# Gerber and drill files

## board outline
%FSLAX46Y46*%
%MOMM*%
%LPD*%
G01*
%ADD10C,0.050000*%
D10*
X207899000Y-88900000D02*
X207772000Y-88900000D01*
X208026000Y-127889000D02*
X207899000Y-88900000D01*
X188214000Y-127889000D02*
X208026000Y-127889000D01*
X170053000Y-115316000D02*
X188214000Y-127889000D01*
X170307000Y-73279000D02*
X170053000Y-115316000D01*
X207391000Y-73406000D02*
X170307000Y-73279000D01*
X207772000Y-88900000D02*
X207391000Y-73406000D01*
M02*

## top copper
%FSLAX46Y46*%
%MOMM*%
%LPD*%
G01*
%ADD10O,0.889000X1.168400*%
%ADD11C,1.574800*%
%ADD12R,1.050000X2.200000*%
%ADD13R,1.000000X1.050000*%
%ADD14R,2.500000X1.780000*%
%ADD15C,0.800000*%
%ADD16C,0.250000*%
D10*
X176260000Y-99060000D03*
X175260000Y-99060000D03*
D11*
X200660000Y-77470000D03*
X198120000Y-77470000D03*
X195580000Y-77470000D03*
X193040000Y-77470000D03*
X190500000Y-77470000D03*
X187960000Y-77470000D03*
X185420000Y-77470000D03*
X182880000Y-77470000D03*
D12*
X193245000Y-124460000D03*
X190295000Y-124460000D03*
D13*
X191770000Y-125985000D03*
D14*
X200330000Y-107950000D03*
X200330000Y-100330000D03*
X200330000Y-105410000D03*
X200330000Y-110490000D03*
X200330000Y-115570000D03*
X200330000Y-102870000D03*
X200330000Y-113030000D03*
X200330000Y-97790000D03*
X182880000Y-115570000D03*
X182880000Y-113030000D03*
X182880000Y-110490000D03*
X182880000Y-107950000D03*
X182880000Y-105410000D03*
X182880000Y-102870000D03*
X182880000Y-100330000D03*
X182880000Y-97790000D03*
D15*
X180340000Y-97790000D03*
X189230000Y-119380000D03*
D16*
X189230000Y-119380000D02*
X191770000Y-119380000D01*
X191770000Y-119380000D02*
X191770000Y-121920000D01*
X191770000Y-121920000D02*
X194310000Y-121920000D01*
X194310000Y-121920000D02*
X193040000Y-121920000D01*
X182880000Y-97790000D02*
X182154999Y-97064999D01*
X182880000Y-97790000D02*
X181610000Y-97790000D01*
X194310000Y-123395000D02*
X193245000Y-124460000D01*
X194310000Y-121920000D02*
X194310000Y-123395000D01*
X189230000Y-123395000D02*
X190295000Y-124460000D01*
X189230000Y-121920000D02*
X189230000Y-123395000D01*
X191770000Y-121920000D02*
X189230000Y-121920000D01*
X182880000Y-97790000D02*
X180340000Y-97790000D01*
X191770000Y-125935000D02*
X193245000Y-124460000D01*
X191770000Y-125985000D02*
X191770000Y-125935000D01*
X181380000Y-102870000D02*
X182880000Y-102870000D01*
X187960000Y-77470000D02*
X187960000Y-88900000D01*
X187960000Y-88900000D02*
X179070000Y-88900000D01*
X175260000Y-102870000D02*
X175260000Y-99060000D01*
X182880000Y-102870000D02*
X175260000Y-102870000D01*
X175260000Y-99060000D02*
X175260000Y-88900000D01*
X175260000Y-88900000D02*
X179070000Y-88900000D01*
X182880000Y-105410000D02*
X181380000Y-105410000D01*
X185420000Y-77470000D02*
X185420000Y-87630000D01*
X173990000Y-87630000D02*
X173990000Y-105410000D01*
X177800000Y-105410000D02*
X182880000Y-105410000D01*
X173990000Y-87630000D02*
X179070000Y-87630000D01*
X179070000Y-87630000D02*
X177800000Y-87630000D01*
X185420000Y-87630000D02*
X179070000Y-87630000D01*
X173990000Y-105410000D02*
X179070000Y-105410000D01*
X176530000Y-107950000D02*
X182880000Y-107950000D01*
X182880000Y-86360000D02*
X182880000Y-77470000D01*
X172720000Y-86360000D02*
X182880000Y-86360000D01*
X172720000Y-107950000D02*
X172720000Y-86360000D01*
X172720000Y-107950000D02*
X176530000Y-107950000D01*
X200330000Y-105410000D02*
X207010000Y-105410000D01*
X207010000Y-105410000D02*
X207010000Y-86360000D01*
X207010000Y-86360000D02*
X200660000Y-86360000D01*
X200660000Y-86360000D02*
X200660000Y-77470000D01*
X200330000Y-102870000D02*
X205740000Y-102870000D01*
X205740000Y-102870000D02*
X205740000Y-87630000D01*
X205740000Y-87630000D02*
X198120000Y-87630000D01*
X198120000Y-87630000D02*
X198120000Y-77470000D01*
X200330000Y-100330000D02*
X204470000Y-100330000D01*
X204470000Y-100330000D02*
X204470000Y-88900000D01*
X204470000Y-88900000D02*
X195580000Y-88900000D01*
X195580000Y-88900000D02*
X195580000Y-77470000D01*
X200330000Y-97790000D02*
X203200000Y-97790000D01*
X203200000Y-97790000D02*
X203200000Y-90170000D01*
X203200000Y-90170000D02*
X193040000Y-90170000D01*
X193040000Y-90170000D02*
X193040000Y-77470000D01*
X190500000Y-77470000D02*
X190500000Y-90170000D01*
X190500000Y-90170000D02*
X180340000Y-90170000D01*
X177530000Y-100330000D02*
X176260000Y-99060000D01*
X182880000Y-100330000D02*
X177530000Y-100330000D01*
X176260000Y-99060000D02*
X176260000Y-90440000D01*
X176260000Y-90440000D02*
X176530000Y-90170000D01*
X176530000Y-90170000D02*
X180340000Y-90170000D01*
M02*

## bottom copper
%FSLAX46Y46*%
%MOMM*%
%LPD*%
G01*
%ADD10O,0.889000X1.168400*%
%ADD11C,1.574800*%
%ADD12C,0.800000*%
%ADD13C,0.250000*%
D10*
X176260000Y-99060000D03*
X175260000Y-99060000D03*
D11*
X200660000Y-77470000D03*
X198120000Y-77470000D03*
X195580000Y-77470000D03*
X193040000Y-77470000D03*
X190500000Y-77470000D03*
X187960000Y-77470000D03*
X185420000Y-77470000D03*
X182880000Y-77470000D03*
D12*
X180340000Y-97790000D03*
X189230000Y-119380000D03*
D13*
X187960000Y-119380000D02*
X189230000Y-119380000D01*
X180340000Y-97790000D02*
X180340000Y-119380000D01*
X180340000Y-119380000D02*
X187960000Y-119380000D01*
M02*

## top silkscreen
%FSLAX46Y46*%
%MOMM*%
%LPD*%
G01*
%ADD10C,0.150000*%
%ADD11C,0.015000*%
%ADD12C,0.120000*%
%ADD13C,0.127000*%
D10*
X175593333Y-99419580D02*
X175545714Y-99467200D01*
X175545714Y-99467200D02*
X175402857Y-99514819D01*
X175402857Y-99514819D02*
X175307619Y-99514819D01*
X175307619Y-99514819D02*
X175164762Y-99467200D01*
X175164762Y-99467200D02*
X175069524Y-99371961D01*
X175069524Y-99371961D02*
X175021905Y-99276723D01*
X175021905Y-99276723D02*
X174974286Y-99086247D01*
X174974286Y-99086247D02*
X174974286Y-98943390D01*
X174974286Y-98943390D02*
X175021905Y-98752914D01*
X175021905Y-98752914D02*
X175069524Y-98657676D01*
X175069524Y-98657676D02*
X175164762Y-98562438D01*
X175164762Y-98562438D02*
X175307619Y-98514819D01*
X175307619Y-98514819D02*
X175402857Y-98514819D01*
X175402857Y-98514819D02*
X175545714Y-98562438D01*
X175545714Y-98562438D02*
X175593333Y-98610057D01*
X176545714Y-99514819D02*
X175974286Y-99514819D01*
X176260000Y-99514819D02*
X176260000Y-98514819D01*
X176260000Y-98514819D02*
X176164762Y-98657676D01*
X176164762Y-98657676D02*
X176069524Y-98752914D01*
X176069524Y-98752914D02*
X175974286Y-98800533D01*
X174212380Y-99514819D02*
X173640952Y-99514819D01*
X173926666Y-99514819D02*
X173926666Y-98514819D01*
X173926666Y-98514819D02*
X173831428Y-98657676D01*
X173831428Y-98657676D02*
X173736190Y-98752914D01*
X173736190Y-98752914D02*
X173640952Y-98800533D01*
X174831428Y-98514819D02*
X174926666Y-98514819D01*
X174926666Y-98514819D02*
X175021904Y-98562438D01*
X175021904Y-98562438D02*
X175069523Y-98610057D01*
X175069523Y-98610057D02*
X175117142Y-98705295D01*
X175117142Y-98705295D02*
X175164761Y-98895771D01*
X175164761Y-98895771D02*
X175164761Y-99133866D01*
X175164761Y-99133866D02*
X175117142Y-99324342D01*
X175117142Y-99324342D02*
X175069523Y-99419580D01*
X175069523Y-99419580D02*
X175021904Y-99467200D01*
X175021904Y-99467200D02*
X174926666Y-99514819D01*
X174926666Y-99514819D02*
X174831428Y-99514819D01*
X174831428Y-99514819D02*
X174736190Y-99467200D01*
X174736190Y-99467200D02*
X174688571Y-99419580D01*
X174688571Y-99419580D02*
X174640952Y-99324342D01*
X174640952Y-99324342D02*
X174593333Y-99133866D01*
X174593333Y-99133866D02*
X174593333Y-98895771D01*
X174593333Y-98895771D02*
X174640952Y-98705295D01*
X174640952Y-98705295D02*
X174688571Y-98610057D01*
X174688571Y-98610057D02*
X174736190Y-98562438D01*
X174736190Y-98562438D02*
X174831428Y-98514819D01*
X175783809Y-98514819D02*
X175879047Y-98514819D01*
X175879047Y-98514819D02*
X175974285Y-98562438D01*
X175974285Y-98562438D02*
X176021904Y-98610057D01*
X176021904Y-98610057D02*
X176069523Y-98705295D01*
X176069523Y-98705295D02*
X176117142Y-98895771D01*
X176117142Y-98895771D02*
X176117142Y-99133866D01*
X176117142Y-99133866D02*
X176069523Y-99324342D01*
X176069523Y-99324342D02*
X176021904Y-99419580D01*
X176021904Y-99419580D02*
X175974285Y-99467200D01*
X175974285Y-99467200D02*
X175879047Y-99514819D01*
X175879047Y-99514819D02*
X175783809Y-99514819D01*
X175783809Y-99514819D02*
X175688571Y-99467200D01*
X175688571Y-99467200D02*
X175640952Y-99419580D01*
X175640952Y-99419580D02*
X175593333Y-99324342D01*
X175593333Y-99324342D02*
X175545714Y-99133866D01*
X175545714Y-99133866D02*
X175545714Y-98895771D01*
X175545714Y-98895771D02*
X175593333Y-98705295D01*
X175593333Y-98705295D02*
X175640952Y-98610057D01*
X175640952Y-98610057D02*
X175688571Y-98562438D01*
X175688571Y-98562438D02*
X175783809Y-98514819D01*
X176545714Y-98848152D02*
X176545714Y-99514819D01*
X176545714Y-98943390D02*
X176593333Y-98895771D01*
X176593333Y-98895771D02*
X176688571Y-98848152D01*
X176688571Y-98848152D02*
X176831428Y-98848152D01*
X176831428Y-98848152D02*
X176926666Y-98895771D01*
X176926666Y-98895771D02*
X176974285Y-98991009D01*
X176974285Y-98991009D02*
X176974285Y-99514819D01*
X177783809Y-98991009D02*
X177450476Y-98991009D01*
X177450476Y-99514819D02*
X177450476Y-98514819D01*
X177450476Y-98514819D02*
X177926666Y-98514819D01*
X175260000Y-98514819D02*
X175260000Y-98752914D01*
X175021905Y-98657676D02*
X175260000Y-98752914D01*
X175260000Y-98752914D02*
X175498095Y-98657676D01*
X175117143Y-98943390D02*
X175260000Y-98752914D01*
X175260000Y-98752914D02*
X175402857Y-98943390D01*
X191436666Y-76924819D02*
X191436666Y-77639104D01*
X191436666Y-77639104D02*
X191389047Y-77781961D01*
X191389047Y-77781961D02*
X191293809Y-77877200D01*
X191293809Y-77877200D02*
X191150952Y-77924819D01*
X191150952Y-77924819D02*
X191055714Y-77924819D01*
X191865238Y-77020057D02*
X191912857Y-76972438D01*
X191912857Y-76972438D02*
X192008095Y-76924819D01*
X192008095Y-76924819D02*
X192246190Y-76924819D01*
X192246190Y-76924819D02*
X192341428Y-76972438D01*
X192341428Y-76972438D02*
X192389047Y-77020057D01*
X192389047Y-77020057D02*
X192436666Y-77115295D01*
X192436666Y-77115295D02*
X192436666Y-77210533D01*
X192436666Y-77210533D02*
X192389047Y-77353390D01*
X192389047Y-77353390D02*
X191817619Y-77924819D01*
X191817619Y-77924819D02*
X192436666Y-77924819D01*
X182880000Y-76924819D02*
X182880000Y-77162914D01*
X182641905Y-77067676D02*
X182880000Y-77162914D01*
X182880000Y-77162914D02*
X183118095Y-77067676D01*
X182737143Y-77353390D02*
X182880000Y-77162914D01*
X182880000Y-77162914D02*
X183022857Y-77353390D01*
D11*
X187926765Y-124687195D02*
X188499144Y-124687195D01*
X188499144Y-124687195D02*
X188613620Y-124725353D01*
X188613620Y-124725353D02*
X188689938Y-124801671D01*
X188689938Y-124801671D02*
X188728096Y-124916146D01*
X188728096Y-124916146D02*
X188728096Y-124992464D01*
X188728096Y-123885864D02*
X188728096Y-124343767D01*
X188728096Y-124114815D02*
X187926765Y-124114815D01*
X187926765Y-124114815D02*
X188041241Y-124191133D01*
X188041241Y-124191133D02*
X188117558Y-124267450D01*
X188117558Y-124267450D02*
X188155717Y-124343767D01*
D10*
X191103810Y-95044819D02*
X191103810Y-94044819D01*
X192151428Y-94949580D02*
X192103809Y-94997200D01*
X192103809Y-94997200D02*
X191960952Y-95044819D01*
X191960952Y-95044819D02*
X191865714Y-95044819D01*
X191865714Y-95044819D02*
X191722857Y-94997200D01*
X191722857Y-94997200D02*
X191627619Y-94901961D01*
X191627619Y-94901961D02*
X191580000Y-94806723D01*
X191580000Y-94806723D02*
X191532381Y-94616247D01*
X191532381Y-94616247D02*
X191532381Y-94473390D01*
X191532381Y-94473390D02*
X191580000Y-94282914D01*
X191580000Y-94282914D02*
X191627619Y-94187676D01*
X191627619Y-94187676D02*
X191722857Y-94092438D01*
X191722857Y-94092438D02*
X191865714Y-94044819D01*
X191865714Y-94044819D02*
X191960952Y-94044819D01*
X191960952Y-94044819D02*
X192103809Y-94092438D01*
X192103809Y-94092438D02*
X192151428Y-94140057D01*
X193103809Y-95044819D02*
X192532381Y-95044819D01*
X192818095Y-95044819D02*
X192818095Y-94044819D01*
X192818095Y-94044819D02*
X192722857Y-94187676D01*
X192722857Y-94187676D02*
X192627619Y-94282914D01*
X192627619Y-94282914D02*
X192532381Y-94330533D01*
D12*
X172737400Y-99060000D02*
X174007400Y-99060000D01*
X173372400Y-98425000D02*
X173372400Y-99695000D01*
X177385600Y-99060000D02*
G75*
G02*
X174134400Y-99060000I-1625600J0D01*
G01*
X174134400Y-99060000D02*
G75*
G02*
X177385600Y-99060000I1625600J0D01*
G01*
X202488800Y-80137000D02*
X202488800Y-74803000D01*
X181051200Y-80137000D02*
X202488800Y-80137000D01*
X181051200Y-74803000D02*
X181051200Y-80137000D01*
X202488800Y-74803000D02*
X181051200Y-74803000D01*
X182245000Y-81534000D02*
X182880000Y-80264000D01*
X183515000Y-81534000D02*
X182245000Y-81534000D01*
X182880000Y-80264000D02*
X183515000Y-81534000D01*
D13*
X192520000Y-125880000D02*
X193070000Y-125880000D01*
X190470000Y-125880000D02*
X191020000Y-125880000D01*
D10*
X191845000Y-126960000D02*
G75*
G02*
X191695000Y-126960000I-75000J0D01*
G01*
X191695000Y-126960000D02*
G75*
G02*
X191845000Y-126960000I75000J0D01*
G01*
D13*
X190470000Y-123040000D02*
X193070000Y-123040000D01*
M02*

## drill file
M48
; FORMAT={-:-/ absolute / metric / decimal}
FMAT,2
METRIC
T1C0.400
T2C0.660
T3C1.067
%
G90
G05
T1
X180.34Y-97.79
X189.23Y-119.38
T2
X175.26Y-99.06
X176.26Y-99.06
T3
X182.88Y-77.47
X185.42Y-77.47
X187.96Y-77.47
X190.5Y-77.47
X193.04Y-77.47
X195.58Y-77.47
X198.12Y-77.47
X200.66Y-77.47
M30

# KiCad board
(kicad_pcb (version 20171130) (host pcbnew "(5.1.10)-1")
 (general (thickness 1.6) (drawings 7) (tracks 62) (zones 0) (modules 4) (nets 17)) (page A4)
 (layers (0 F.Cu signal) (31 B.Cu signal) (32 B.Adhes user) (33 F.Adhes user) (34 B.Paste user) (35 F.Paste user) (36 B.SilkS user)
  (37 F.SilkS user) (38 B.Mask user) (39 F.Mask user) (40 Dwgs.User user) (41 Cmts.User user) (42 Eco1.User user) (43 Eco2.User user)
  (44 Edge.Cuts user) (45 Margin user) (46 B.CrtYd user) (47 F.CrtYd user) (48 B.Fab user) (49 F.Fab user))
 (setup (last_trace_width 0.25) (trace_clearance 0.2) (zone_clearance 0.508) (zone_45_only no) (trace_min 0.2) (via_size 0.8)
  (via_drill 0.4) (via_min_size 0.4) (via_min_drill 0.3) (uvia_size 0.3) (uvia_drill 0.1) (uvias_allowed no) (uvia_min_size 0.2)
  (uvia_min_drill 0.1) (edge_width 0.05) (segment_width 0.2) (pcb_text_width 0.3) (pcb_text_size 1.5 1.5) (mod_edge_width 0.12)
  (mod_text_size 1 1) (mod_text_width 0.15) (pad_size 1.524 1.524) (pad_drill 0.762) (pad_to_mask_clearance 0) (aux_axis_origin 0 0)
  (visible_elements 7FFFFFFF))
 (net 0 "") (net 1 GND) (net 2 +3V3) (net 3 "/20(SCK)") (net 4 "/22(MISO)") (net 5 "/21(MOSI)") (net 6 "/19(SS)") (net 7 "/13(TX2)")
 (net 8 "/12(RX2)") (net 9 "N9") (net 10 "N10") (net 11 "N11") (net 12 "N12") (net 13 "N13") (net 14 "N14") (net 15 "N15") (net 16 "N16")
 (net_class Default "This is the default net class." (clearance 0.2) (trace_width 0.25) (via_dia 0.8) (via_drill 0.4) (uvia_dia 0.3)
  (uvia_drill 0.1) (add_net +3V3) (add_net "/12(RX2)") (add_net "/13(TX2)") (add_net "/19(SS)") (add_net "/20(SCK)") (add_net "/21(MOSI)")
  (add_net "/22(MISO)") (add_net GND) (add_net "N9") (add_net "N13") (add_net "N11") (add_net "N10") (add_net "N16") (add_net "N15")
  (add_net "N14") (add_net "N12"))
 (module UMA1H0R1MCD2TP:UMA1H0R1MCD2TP (layer F.Cu) (at 175.26 99.06)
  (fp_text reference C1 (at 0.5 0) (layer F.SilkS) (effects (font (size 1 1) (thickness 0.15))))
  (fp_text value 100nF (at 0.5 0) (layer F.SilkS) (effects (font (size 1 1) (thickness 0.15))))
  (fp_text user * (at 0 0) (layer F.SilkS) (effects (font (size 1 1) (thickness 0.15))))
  (fp_line (start -2.5226 0) (end -1.2526 0) (layer F.SilkS) (width 0.12))
  (fp_line (start -1.8876 -0.635) (end -1.8876 0.635) (layer F.SilkS) (width 0.12))
  (fp_circle (center 0.5 0) (end 2.1256 0) (layer F.SilkS) (width 0.12))
  (pad 2 thru_hole oval (at 1 0) (size 0.889 1.1684) (drill 0.6604) (layers *.Cu *.Mask) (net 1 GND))
  (pad 1 thru_hole oval (at 0 0) (size 0.889 1.1684) (drill 0.6604) (layers *.Cu *.Mask) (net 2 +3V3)))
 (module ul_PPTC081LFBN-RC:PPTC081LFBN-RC (layer F.Cu) (at 182.88 77.47 180)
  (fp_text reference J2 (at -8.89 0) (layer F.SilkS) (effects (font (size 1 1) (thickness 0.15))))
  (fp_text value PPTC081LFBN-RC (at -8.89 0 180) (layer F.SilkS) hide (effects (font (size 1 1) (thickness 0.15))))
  (fp_line (start -19.6088 -2.667) (end -19.6088 2.667) (layer F.SilkS) (width 0.12))
  (fp_line (start 1.8288 -2.667) (end -19.6088 -2.667) (layer F.SilkS) (width 0.12))
  (fp_line (start 1.8288 2.667) (end 1.8288 -2.667) (layer F.SilkS) (width 0.12))
  (fp_line (start -19.6088 2.667) (end 1.8288 2.667) (layer F.SilkS) (width 0.12))
  (fp_line (start 0.635 -4.064) (end 0 -2.794) (layer F.SilkS) (width 0.12))
  (fp_line (start -0.635 -4.064) (end 0.635 -4.064) (layer F.SilkS) (width 0.12))
  (fp_line (start 0 -2.794) (end -0.635 -4.064) (layer F.SilkS) (width 0.12))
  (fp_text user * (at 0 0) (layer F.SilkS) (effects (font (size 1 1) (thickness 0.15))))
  (pad 8 thru_hole circle (at -17.78 0 180) (size 1.5748 1.5748) (drill 1.0668) (layers *.Cu *.Mask) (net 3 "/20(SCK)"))
  (pad 7 thru_hole circle (at -15.24 0 180) (size 1.5748 1.5748) (drill 1.0668) (layers *.Cu *.Mask) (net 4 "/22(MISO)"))
  (pad 6 thru_hole circle (at -12.7 0 180) (size 1.5748 1.5748) (drill 1.0668) (layers *.Cu *.Mask) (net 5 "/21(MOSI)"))
  (pad 5 thru_hole circle (at -10.16 0 180) (size 1.5748 1.5748) (drill 1.0668) (layers *.Cu *.Mask) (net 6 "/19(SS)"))
  (pad 4 thru_hole circle (at -7.62 0 180) (size 1.5748 1.5748) (drill 1.0668) (layers *.Cu *.Mask) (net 1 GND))
  (pad 3 thru_hole circle (at -5.08 0 180) (size 1.5748 1.5748) (drill 1.0668) (layers *.Cu *.Mask) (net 2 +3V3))
  (pad 2 thru_hole circle (at -2.54 0 180) (size 1.5748 1.5748) (drill 1.0668) (layers *.Cu *.Mask) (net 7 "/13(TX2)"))
  (pad 1 thru_hole circle (at 0 0 180) (size 1.5748 1.5748) (drill 1.0668) (layers *.Cu *.Mask) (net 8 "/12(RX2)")))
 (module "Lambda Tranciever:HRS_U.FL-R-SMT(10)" (layer F.Cu) (at 191.77 124.46 90)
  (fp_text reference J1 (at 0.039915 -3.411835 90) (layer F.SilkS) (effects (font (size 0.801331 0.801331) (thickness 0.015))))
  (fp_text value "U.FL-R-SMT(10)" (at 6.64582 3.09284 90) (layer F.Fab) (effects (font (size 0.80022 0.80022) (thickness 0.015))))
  (fp_line (start -1.42 0.75) (end -1.42 1.3) (layer F.SilkS) (width 0.127))
  (fp_line (start -1.42 -1.3) (end -1.42 -0.75) (layer F.SilkS) (width 0.127))
  (fp_circle (center -2.5 0) (end -2.425 0) (layer F.SilkS) (width 0.15))
  (fp_line (start 1.42 -1.3) (end 1.42 1.3) (layer F.SilkS) (width 0.127))
  (pad 3 smd rect (at 0 1.475 90) (size 2.2 1.05) (layers F.Cu F.Paste F.Mask) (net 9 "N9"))
  (pad 2 smd rect (at 0 -1.475 90) (size 2.2 1.05) (layers F.Cu F.Paste F.Mask) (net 9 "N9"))
  (pad 1 smd rect (at -1.525 0 90) (size 1.05 1) (layers F.Cu F.Paste F.Mask) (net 9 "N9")))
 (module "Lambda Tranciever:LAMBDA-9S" (layer F.Cu) (at 182.88 97.79)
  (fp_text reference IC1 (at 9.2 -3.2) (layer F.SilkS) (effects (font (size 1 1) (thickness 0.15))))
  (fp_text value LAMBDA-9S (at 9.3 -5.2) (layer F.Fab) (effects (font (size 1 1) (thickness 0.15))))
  (pad 12 smd rect (at 17.45 10.16) (size 2.5 1.78) (layers F.Cu F.Paste F.Mask) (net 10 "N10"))
  (pad 15 smd rect (at 17.45 2.54) (size 2.5 1.78) (layers F.Cu F.Paste F.Mask) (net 5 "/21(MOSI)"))
  (pad 13 smd rect (at 17.45 7.62) (size 2.5 1.78) (layers F.Cu F.Paste F.Mask) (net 3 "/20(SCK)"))
  (pad 11 smd rect (at 17.45 12.7) (size 2.5 1.78) (layers F.Cu F.Paste F.Mask) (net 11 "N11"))
  (pad 9 smd rect (at 17.45 17.78) (size 2.5 1.78) (layers F.Cu F.Paste F.Mask) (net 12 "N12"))
  (pad 14 smd rect (at 17.45 5.08) (size 2.5 1.78) (layers F.Cu F.Paste F.Mask) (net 4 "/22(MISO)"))
  (pad 10 smd rect (at 17.45 15.24) (size 2.5 1.78) (layers F.Cu F.Paste F.Mask) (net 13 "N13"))
  (pad 16 smd rect (at 17.45 0) (size 2.5 1.78) (layers F.Cu F.Paste F.Mask) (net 6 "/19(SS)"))
  (pad 8 smd rect (at 0 17.78) (size 2.5 1.78) (layers F.Cu F.Paste F.Mask) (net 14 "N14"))
  (pad 7 smd rect (at 0 15.24) (size 2.5 1.78) (layers F.Cu F.Paste F.Mask) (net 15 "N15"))
  (pad 6 smd rect (at 0 12.7) (size 2.5 1.78) (layers F.Cu F.Paste F.Mask) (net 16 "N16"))
  (pad 5 smd rect (at 0 10.16) (size 2.5 1.78) (layers F.Cu F.Paste F.Mask) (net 8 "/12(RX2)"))
  (pad 4 smd rect (at 0 7.62) (size 2.5 1.78) (layers F.Cu F.Paste F.Mask) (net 7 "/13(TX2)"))
  (pad 3 smd rect (at 0 5.08) (size 2.5 1.78) (layers F.Cu F.Paste F.Mask) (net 2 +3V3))
  (pad 2 smd rect (at 0 2.54) (size 2.5 1.78) (layers F.Cu F.Paste F.Mask) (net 1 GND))
  (pad 1 smd rect (at 0 0) (size 2.5 1.78) (layers F.Cu F.Paste F.Mask) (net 9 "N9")))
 (gr_line (start 207.899 88.9) (end 207.772 88.9) (layer Edge.Cuts) (width 0.05))
 (gr_line (start 208.026 127.889) (end 207.899 88.9) (layer Edge.Cuts) (width 0.05))
 (gr_line (start 188.214 127.889) (end 208.026 127.889) (layer Edge.Cuts) (width 0.05))
 (gr_line (start 170.053 115.316) (end 188.214 127.889) (layer Edge.Cuts) (width 0.05))
 (gr_line (start 170.307 73.279) (end 170.053 115.316) (layer Edge.Cuts) (width 0.05))
 (gr_line (start 207.391 73.406) (end 170.307 73.279) (layer Edge.Cuts) (width 0.05))
 (gr_line (start 207.772 88.9) (end 207.391 73.406) (layer Edge.Cuts) (width 0.05))
 (via (at 180.34 97.79) (size 0.8) (drill 0.4) (layers F.Cu B.Cu) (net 9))
 (via (at 189.23 119.38) (size 0.8) (drill 0.4) (layers F.Cu B.Cu) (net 9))
 (segment (start 189.23 119.38) (end 191.77 119.38) (width 0.25) (layer F.Cu) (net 9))
 (segment (start 191.77 119.38) (end 191.77 121.92) (width 0.25) (layer F.Cu) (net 9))
 (segment (start 191.77 121.92) (end 194.31 121.92) (width 0.25) (layer F.Cu) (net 9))
 (segment (start 194.31 121.92) (end 193.04 121.92) (width 0.25) (layer F.Cu) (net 9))
 (segment (start 182.88 97.79) (end 182.154999 97.064999) (width 0.25) (layer F.Cu) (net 9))
 (segment (start 182.88 97.79) (end 181.61 97.79) (width 0.25) (layer F.Cu) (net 9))
 (segment (start 187.96 119.38) (end 189.23 119.38) (width 0.25) (layer B.Cu) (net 9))
 (segment (start 194.31 123.395) (end 193.245 124.46) (width 0.25) (layer F.Cu) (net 9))
 (segment (start 194.31 121.92) (end 194.31 123.395) (width 0.25) (layer F.Cu) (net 9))
 (segment (start 189.23 123.395) (end 190.295 124.46) (width 0.25) (layer F.Cu) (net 9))
 (segment (start 189.23 121.92) (end 189.23 123.395) (width 0.25) (layer F.Cu) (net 9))
 (segment (start 191.77 121.92) (end 189.23 121.92) (width 0.25) (layer F.Cu) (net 9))
 (segment (start 182.88 97.79) (end 180.34 97.79) (width 0.25) (layer F.Cu) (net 9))
 (segment (start 180.34 97.79) (end 180.34 119.38) (width 0.25) (layer B.Cu) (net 9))
 (segment (start 180.34 119.38) (end 187.96 119.38) (width 0.25) (layer B.Cu) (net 9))
 (segment (start 191.77 125.935) (end 193.245 124.46) (width 0.25) (layer F.Cu) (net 9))
 (segment (start 191.77 125.985) (end 191.77 125.935) (width 0.25) (layer F.Cu) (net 9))
 (segment (start 181.38 102.87) (end 182.88 102.87) (width 0.25) (layer F.Cu) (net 2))
 (segment (start 187.96 77.47) (end 187.96 88.9) (width 0.25) (layer F.Cu) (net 2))
 (segment (start 187.96 88.9) (end 179.07 88.9) (width 0.25) (layer F.Cu) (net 2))
 (segment (start 175.26 102.87) (end 175.26 99.06) (width 0.25) (layer F.Cu) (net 2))
 (segment (start 182.88 102.87) (end 175.26 102.87) (width 0.25) (layer F.Cu) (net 2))
 (segment (start 175.26 99.06) (end 175.26 88.9) (width 0.25) (layer F.Cu) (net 2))
 (segment (start 175.26 88.9) (end 179.07 88.9) (width 0.25) (layer F.Cu) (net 2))
 (segment (start 182.88 105.41) (end 181.38 105.41) (width 0.25) (layer F.Cu) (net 7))
 (segment (start 185.42 77.47) (end 185.42 87.63) (width 0.25) (layer F.Cu) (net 7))
 (segment (start 173.99 87.63) (end 173.99 105.41) (width 0.25) (layer F.Cu) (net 7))
 (segment (start 177.8 105.41) (end 182.88 105.41) (width 0.25) (layer F.Cu) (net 7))
 (segment (start 173.99 87.63) (end 179.07 87.63) (width 0.25) (layer F.Cu) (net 7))
 (segment (start 179.07 87.63) (end 177.8 87.63) (width 0.25) (layer F.Cu) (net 7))
 (segment (start 185.42 87.63) (end 179.07 87.63) (width 0.25) (layer F.Cu) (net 7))
 (segment (start 173.99 105.41) (end 179.07 105.41) (width 0.25) (layer F.Cu) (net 7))
 (segment (start 176.53 107.95) (end 182.88 107.95) (width 0.25) (layer F.Cu) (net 8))
 (segment (start 182.88 86.36) (end 182.88 77.47) (width 0.25) (layer F.Cu) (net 8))
 (segment (start 172.72 86.36) (end 182.88 86.36) (width 0.25) (layer F.Cu) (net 8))
 (segment (start 172.72 107.95) (end 172.72 86.36) (width 0.25) (layer F.Cu) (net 8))
 (segment (start 172.72 107.95) (end 176.53 107.95) (width 0.25) (layer F.Cu) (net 8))
 (segment (start 200.33 105.41) (end 207.01 105.41) (width 0.25) (layer F.Cu) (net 3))
 (segment (start 207.01 105.41) (end 207.01 86.36) (width 0.25) (layer F.Cu) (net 3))
 (segment (start 207.01 86.36) (end 200.66 86.36) (width 0.25) (layer F.Cu) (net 3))
 (segment (start 200.66 86.36) (end 200.66 77.47) (width 0.25) (layer F.Cu) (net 3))
 (segment (start 200.33 102.87) (end 205.74 102.87) (width 0.25) (layer F.Cu) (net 4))
 (segment (start 205.74 102.87) (end 205.74 87.63) (width 0.25) (layer F.Cu) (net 4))
 (segment (start 205.74 87.63) (end 198.12 87.63) (width 0.25) (layer F.Cu) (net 4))
 (segment (start 198.12 87.63) (end 198.12 77.47) (width 0.25) (layer F.Cu) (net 4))
 (segment (start 200.33 100.33) (end 204.47 100.33) (width 0.25) (layer F.Cu) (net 5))
 (segment (start 204.47 100.33) (end 204.47 88.9) (width 0.25) (layer F.Cu) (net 5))
 (segment (start 204.47 88.9) (end 195.58 88.9) (width 0.25) (layer F.Cu) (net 5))
 (segment (start 195.58 88.9) (end 195.58 77.47) (width 0.25) (layer F.Cu) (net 5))
 (segment (start 200.33 97.79) (end 203.2 97.79) (width 0.25) (layer F.Cu) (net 6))
 (segment (start 203.2 97.79) (end 203.2 90.17) (width 0.25) (layer F.Cu) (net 6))
 (segment (start 203.2 90.17) (end 193.04 90.17) (width 0.25) (layer F.Cu) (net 6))
 (segment (start 193.04 90.17) (end 193.04 77.47) (width 0.25) (layer F.Cu) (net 6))
 (segment (start 190.5 77.47) (end 190.5 90.17) (width 0.25) (layer F.Cu) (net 1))
 (segment (start 190.5 90.17) (end 180.34 90.17) (width 0.25) (layer F.Cu) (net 1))
 (segment (start 177.53 100.33) (end 176.26 99.06) (width 0.25) (layer F.Cu) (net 1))
 (segment (start 182.88 100.33) (end 177.53 100.33) (width 0.25) (layer F.Cu) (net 1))
 (segment (start 176.26 99.06) (end 176.26 90.44) (width 0.25) (layer F.Cu) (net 1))
 (segment (start 176.26 90.44) (end 176.53 90.17) (width 0.25) (layer F.Cu) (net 1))
 (segment (start 176.53 90.17) (end 180.34 90.17) (width 0.25) (layer F.Cu) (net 1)))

